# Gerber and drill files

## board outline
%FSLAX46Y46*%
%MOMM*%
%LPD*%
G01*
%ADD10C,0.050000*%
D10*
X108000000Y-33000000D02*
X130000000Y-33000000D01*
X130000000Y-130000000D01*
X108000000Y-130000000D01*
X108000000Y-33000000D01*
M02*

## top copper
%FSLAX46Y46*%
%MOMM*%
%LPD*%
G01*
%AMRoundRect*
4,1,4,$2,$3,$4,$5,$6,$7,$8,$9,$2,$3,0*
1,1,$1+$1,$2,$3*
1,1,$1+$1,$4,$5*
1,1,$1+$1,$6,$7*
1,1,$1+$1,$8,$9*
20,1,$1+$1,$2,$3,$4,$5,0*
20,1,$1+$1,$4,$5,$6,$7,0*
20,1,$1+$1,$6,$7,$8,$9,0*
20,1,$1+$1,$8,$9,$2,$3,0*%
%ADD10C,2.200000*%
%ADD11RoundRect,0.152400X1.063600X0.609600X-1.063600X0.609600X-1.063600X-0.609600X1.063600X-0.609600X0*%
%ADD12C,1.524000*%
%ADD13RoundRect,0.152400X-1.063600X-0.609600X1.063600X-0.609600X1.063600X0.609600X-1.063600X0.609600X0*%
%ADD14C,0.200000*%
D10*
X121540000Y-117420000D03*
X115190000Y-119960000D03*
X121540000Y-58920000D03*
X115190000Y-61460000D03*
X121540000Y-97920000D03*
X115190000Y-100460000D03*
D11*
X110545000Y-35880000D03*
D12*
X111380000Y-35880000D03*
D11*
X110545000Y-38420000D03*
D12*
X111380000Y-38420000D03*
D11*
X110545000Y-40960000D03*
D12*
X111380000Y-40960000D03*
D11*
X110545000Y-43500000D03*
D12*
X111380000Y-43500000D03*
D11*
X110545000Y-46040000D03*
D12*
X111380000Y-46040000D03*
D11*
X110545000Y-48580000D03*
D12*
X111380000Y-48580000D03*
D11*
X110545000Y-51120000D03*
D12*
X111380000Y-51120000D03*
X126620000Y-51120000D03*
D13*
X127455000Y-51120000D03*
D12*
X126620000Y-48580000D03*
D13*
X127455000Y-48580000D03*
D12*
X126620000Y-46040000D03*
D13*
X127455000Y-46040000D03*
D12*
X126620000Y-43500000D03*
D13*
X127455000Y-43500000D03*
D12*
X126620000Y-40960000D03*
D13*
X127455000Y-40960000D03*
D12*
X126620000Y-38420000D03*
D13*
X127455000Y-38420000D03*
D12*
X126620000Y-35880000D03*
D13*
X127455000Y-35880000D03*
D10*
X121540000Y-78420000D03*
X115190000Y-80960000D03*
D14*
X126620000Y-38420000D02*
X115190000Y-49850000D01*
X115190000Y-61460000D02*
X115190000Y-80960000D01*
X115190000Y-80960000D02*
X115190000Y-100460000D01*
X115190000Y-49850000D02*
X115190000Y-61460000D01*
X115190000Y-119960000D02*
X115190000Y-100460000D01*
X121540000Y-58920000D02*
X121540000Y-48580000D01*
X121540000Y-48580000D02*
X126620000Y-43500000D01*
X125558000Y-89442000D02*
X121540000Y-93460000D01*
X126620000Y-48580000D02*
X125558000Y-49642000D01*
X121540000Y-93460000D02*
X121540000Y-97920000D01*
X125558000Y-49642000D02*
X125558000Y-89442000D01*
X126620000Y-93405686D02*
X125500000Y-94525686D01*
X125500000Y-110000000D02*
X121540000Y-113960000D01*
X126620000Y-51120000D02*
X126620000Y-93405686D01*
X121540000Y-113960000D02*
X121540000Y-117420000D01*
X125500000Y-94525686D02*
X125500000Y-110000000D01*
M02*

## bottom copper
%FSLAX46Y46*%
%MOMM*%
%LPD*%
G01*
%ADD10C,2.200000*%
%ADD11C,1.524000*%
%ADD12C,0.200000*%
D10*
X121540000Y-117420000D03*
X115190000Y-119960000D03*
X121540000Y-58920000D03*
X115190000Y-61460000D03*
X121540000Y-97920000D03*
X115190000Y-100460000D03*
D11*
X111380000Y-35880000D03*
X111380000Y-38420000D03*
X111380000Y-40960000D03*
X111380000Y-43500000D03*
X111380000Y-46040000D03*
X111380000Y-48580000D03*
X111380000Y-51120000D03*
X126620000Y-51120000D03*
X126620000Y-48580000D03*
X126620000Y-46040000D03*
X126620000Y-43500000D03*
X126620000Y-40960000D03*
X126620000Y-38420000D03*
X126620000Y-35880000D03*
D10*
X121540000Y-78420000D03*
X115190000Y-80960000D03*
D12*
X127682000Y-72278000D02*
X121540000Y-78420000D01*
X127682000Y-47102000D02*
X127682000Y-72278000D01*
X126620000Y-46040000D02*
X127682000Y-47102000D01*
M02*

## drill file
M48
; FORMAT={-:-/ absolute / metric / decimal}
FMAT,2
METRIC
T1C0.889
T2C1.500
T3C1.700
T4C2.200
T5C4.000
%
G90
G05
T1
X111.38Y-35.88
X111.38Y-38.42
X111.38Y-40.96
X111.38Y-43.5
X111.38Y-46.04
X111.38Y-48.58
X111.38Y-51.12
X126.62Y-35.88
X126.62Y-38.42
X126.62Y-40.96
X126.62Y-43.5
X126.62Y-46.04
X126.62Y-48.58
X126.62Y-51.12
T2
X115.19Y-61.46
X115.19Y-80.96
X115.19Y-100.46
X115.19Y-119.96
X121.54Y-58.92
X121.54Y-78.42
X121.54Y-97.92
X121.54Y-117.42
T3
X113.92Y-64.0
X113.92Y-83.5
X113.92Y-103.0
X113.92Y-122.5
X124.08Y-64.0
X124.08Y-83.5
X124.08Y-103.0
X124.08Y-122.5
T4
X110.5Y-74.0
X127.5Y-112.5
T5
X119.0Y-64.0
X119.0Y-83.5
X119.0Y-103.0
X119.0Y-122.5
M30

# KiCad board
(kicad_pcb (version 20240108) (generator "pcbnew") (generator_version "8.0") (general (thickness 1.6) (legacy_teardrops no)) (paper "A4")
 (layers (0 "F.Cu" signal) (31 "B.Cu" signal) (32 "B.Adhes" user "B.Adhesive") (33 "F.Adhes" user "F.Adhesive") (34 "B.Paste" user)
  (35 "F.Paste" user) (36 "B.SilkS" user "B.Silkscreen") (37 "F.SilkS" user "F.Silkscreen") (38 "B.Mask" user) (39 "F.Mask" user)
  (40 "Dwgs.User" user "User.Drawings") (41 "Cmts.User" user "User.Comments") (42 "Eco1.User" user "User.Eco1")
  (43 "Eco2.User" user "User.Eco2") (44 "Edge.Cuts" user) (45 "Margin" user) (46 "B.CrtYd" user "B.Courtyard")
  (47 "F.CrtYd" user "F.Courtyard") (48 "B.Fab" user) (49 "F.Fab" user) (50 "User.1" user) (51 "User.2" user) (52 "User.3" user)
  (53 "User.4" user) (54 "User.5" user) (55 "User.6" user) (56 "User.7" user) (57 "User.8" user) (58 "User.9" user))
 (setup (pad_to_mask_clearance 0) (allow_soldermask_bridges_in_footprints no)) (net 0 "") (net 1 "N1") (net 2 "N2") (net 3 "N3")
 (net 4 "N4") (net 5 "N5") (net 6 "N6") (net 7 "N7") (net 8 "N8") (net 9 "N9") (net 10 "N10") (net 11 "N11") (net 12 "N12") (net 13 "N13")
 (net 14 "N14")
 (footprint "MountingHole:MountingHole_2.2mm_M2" (layer "F.Cu") (at 110.5 74)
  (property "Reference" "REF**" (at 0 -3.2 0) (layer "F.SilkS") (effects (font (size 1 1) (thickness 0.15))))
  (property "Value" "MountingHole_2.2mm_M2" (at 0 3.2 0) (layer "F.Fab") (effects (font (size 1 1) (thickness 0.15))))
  (pad "" np_thru_hole circle (at 0 0) (size 2.2 2.2) (drill 2.2) (layers "*.Cu" "*.Mask")))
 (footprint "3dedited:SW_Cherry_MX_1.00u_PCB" (layer "F.Cu") (at 121.54 117.42)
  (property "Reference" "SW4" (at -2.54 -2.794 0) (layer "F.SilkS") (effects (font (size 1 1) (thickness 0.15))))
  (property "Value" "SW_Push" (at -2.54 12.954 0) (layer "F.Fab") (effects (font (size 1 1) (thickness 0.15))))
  (pad "" np_thru_hole circle (at -7.62 5.08) (size 1.7 1.7) (drill 1.7) (layers "*.Cu" "*.Mask"))
  (pad "" np_thru_hole circle (at -2.54 5.08) (size 4 4) (drill 4) (layers "*.Cu" "*.Mask"))
  (pad "" np_thru_hole circle (at 2.54 5.08) (size 1.7 1.7) (drill 1.7) (layers "*.Cu" "*.Mask"))
  (pad "1" thru_hole circle (at 0 0) (size 2.2 2.2) (drill 1.5) (layers "*.Cu" "*.Mask") (remove_unused_layers no) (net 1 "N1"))
  (pad "2" thru_hole circle (at -6.35 2.54) (size 2.2 2.2) (drill 1.5) (layers "*.Cu" "*.Mask") (remove_unused_layers no) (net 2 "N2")))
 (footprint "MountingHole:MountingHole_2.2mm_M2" (layer "F.Cu") (at 127.5 112.5)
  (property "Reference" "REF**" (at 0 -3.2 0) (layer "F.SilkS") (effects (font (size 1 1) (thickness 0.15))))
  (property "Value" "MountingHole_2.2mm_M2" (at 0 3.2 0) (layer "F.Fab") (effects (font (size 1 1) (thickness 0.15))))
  (pad "" np_thru_hole circle (at 0 0) (size 2.2 2.2) (drill 2.2) (layers "*.Cu" "*.Mask")))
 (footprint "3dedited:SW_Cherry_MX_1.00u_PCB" (layer "F.Cu") (at 121.54 58.92)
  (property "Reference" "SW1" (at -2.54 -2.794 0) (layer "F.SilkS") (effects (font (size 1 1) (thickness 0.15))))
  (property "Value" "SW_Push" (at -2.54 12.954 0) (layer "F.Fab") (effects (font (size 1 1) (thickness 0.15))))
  (pad "" np_thru_hole circle (at -7.62 5.08) (size 1.7 1.7) (drill 1.7) (layers "*.Cu" "*.Mask"))
  (pad "" np_thru_hole circle (at -2.54 5.08) (size 4 4) (drill 4) (layers "*.Cu" "*.Mask"))
  (pad "" np_thru_hole circle (at 2.54 5.08) (size 1.7 1.7) (drill 1.7) (layers "*.Cu" "*.Mask"))
  (pad "1" thru_hole circle (at 0 0) (size 2.2 2.2) (drill 1.5) (layers "*.Cu" "*.Mask") (remove_unused_layers no) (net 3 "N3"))
  (pad "2" thru_hole circle (at -6.35 2.54) (size 2.2 2.2) (drill 1.5) (layers "*.Cu" "*.Mask") (remove_unused_layers no) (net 2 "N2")))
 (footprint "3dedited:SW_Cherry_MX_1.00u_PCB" (layer "F.Cu") (at 121.54 97.92)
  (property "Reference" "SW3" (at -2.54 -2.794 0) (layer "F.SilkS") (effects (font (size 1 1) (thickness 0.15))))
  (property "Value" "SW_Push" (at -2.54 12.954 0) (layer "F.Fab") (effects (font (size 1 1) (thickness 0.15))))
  (pad "" np_thru_hole circle (at -7.62 5.08) (size 1.7 1.7) (drill 1.7) (layers "*.Cu" "*.Mask"))
  (pad "" np_thru_hole circle (at -2.54 5.08) (size 4 4) (drill 4) (layers "*.Cu" "*.Mask"))
  (pad "" np_thru_hole circle (at 2.54 5.08) (size 1.7 1.7) (drill 1.7) (layers "*.Cu" "*.Mask"))
  (pad "1" thru_hole circle (at 0 0) (size 2.2 2.2) (drill 1.5) (layers "*.Cu" "*.Mask") (remove_unused_layers no) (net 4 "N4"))
  (pad "2" thru_hole circle (at -6.35 2.54) (size 2.2 2.2) (drill 1.5) (layers "*.Cu" "*.Mask") (remove_unused_layers no) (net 2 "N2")))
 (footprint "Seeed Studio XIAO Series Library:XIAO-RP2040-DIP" (layer "F.Cu") (at 119 43.5)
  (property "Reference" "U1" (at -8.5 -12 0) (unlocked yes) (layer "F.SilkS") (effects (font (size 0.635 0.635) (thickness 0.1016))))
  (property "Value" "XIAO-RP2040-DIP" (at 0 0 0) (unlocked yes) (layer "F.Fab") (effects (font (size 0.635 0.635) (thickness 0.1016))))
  (pad "1" smd roundrect (at -8.455 -7.62 180) (size 2.432 1.524) (layers "F.Cu" "F.Mask") (roundrect_rratio 0.1) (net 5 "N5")
   (thermal_bridge_angle 45))
  (pad "1" thru_hole circle (at -7.62 -7.62 180) (size 1.524 1.524) (drill 0.889) (layers "*.Cu" "*.Mask") (remove_unused_layers no)
   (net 5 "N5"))
  (pad "2" smd roundrect (at -8.455 -5.08 180) (size 2.432 1.524) (layers "F.Cu" "F.Mask") (roundrect_rratio 0.1) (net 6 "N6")
   (thermal_bridge_angle 45))
  (pad "2" thru_hole circle (at -7.62 -5.08 180) (size 1.524 1.524) (drill 0.889) (layers "*.Cu" "*.Mask") (remove_unused_layers no)
   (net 6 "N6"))
  (pad "3" smd roundrect (at -8.455 -2.54 180) (size 2.432 1.524) (layers "F.Cu" "F.Mask") (roundrect_rratio 0.1) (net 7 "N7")
   (thermal_bridge_angle 45))
  (pad "3" thru_hole circle (at -7.62 -2.54 180) (size 1.524 1.524) (drill 0.889) (layers "*.Cu" "*.Mask") (remove_unused_layers no)
   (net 7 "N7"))
  (pad "4" smd roundrect (at -8.455 0 180) (size 2.432 1.524) (layers "F.Cu" "F.Mask") (roundrect_rratio 0.1) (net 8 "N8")
   (thermal_bridge_angle 45))
  (pad "4" thru_hole circle (at -7.62 0 180) (size 1.524 1.524) (drill 0.889) (layers "*.Cu" "*.Mask") (remove_unused_layers no)
   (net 8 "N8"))
  (pad "5" smd roundrect (at -8.455 2.54 180) (size 2.432 1.524) (layers "F.Cu" "F.Mask") (roundrect_rratio 0.1) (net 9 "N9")
   (thermal_bridge_angle 45))
  (pad "5" thru_hole circle (at -7.62 2.54 180) (size 1.524 1.524) (drill 0.889) (layers "*.Cu" "*.Mask") (remove_unused_layers no)
   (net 9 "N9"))
  (pad "6" smd roundrect (at -8.455 5.08 180) (size 2.432 1.524) (layers "F.Cu" "F.Mask") (roundrect_rratio 0.1) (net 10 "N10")
   (thermal_bridge_angle 45))
  (pad "6" thru_hole circle (at -7.62 5.08 180) (size 1.524 1.524) (drill 0.889) (layers "*.Cu" "*.Mask") (remove_unused_layers no)
   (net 10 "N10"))
  (pad "7" smd roundrect (at -8.455 7.62 180) (size 2.432 1.524) (layers "F.Cu" "F.Mask") (roundrect_rratio 0.1) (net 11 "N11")
   (thermal_bridge_angle 45))
  (pad "7" thru_hole circle (at -7.62 7.62 180) (size 1.524 1.524) (drill 0.889) (layers "*.Cu" "*.Mask") (remove_unused_layers no)
   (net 11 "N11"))
  (pad "8" thru_hole circle (at 7.62 7.62) (size 1.524 1.524) (drill 0.889) (layers "*.Cu" "*.Mask") (remove_unused_layers no) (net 1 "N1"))
  (pad "8" smd roundrect (at 8.455 7.62) (size 2.432 1.524) (layers "F.Cu" "F.Mask") (roundrect_rratio 0.1) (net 1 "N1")
   (thermal_bridge_angle 45))
  (pad "9" thru_hole circle (at 7.62 5.08) (size 1.524 1.524) (drill 0.889) (layers "*.Cu" "*.Mask") (remove_unused_layers no) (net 4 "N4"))
  (pad "9" smd roundrect (at 8.455 5.08) (size 2.432 1.524) (layers "F.Cu" "F.Mask") (roundrect_rratio 0.1) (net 4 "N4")
   (thermal_bridge_angle 45))
  (pad "10" thru_hole circle (at 7.62 2.54) (size 1.524 1.524) (drill 0.889) (layers "*.Cu" "*.Mask") (remove_unused_layers no)
   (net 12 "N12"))
  (pad "10" smd roundrect (at 8.455 2.54) (size 2.432 1.524) (layers "F.Cu" "F.Mask") (roundrect_rratio 0.1) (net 12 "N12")
   (thermal_bridge_angle 45))
  (pad "11" thru_hole circle (at 7.62 0) (size 1.524 1.524) (drill 0.889) (layers "*.Cu" "*.Mask") (remove_unused_layers no) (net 3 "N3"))
  (pad "11" smd roundrect (at 8.455 0) (size 2.432 1.524) (layers "F.Cu" "F.Mask") (roundrect_rratio 0.1) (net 3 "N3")
   (thermal_bridge_angle 45))
  (pad "12" thru_hole circle (at 7.62 -2.54) (size 1.524 1.524) (drill 0.889) (layers "*.Cu" "*.Mask") (remove_unused_layers no)
   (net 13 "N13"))
  (pad "12" smd roundrect (at 8.455 -2.54) (size 2.432 1.524) (layers "F.Cu" "F.Mask") (roundrect_rratio 0.1) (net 13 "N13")
   (thermal_bridge_angle 45))
  (pad "13" thru_hole circle (at 7.62 -5.08) (size 1.524 1.524) (drill 0.889) (layers "*.Cu" "*.Mask") (remove_unused_layers no)
   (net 2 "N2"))
  (pad "13" smd roundrect (at 8.455 -5.08) (size 2.432 1.524) (layers "F.Cu" "F.Mask") (roundrect_rratio 0.1) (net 2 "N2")
   (thermal_bridge_angle 45))
  (pad "14" thru_hole circle (at 7.62 -7.62) (size 1.524 1.524) (drill 0.889) (layers "*.Cu" "*.Mask") (remove_unused_layers no)
   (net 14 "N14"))
  (pad "14" smd roundrect (at 8.455 -7.62) (size 2.432 1.524) (layers "F.Cu" "F.Mask") (roundrect_rratio 0.1) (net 14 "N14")
   (thermal_bridge_angle 45)))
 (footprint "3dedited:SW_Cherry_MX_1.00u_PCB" (layer "F.Cu") (at 121.54 78.42)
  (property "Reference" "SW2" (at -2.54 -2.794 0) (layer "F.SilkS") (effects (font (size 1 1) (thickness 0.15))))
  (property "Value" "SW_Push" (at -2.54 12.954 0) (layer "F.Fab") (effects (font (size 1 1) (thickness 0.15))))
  (pad "" np_thru_hole circle (at -7.62 5.08) (size 1.7 1.7) (drill 1.7) (layers "*.Cu" "*.Mask"))
  (pad "" np_thru_hole circle (at -2.54 5.08) (size 4 4) (drill 4) (layers "*.Cu" "*.Mask"))
  (pad "" np_thru_hole circle (at 2.54 5.08) (size 1.7 1.7) (drill 1.7) (layers "*.Cu" "*.Mask"))
  (pad "1" thru_hole circle (at 0 0) (size 2.2 2.2) (drill 1.5) (layers "*.Cu" "*.Mask") (remove_unused_layers no) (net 12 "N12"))
  (pad "2" thru_hole circle (at -6.35 2.54) (size 2.2 2.2) (drill 1.5) (layers "*.Cu" "*.Mask") (remove_unused_layers no) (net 2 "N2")))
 (gr_rect (start 108 33) (end 130 130) (stroke (width 0.05) (type default)) (fill none) (layer "Edge.Cuts"))
 (segment (start 126.62 38.42) (end 115.19 49.85) (width 0.2) (layer "F.Cu") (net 2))
 (segment (start 115.19 61.46) (end 115.19 80.96) (width 0.2) (layer "F.Cu") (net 2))
 (segment (start 115.19 80.96) (end 115.19 100.46) (width 0.2) (layer "F.Cu") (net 2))
 (segment (start 115.19 49.85) (end 115.19 61.46) (width 0.2) (layer "F.Cu") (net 2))
 (segment (start 115.19 119.96) (end 115.19 100.46) (width 0.2) (layer "F.Cu") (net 2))
 (segment (start 121.54 58.92) (end 121.54 48.58) (width 0.2) (layer "F.Cu") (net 3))
 (segment (start 121.54 48.58) (end 126.62 43.5) (width 0.2) (layer "F.Cu") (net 3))
 (segment (start 127.682 72.278) (end 121.54 78.42) (width 0.2) (layer "B.Cu") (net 12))
 (segment (start 127.682 47.102) (end 127.682 72.278) (width 0.2) (layer "B.Cu") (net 12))
 (segment (start 126.62 46.04) (end 127.682 47.102) (width 0.2) (layer "B.Cu") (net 12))
 (segment (start 125.558 89.442) (end 121.54 93.46) (width 0.2) (layer "F.Cu") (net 4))
 (segment (start 126.62 48.58) (end 125.558 49.642) (width 0.2) (layer "F.Cu") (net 4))
 (segment (start 121.54 93.46) (end 121.54 97.92) (width 0.2) (layer "F.Cu") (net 4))
 (segment (start 125.558 49.642) (end 125.558 89.442) (width 0.2) (layer "F.Cu") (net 4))
 (segment (start 126.62 93.405686) (end 125.5 94.525686) (width 0.2) (layer "F.Cu") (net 1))
 (segment (start 125.5 110) (end 121.54 113.96) (width 0.2) (layer "F.Cu") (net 1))
 (segment (start 126.62 51.12) (end 126.62 93.405686) (width 0.2) (layer "F.Cu") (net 1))
 (segment (start 121.54 113.96) (end 121.54 117.42) (width 0.2) (layer "F.Cu") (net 1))
 (segment (start 125.5 94.525686) (end 125.5 110) (width 0.2) (layer "F.Cu") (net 1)))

